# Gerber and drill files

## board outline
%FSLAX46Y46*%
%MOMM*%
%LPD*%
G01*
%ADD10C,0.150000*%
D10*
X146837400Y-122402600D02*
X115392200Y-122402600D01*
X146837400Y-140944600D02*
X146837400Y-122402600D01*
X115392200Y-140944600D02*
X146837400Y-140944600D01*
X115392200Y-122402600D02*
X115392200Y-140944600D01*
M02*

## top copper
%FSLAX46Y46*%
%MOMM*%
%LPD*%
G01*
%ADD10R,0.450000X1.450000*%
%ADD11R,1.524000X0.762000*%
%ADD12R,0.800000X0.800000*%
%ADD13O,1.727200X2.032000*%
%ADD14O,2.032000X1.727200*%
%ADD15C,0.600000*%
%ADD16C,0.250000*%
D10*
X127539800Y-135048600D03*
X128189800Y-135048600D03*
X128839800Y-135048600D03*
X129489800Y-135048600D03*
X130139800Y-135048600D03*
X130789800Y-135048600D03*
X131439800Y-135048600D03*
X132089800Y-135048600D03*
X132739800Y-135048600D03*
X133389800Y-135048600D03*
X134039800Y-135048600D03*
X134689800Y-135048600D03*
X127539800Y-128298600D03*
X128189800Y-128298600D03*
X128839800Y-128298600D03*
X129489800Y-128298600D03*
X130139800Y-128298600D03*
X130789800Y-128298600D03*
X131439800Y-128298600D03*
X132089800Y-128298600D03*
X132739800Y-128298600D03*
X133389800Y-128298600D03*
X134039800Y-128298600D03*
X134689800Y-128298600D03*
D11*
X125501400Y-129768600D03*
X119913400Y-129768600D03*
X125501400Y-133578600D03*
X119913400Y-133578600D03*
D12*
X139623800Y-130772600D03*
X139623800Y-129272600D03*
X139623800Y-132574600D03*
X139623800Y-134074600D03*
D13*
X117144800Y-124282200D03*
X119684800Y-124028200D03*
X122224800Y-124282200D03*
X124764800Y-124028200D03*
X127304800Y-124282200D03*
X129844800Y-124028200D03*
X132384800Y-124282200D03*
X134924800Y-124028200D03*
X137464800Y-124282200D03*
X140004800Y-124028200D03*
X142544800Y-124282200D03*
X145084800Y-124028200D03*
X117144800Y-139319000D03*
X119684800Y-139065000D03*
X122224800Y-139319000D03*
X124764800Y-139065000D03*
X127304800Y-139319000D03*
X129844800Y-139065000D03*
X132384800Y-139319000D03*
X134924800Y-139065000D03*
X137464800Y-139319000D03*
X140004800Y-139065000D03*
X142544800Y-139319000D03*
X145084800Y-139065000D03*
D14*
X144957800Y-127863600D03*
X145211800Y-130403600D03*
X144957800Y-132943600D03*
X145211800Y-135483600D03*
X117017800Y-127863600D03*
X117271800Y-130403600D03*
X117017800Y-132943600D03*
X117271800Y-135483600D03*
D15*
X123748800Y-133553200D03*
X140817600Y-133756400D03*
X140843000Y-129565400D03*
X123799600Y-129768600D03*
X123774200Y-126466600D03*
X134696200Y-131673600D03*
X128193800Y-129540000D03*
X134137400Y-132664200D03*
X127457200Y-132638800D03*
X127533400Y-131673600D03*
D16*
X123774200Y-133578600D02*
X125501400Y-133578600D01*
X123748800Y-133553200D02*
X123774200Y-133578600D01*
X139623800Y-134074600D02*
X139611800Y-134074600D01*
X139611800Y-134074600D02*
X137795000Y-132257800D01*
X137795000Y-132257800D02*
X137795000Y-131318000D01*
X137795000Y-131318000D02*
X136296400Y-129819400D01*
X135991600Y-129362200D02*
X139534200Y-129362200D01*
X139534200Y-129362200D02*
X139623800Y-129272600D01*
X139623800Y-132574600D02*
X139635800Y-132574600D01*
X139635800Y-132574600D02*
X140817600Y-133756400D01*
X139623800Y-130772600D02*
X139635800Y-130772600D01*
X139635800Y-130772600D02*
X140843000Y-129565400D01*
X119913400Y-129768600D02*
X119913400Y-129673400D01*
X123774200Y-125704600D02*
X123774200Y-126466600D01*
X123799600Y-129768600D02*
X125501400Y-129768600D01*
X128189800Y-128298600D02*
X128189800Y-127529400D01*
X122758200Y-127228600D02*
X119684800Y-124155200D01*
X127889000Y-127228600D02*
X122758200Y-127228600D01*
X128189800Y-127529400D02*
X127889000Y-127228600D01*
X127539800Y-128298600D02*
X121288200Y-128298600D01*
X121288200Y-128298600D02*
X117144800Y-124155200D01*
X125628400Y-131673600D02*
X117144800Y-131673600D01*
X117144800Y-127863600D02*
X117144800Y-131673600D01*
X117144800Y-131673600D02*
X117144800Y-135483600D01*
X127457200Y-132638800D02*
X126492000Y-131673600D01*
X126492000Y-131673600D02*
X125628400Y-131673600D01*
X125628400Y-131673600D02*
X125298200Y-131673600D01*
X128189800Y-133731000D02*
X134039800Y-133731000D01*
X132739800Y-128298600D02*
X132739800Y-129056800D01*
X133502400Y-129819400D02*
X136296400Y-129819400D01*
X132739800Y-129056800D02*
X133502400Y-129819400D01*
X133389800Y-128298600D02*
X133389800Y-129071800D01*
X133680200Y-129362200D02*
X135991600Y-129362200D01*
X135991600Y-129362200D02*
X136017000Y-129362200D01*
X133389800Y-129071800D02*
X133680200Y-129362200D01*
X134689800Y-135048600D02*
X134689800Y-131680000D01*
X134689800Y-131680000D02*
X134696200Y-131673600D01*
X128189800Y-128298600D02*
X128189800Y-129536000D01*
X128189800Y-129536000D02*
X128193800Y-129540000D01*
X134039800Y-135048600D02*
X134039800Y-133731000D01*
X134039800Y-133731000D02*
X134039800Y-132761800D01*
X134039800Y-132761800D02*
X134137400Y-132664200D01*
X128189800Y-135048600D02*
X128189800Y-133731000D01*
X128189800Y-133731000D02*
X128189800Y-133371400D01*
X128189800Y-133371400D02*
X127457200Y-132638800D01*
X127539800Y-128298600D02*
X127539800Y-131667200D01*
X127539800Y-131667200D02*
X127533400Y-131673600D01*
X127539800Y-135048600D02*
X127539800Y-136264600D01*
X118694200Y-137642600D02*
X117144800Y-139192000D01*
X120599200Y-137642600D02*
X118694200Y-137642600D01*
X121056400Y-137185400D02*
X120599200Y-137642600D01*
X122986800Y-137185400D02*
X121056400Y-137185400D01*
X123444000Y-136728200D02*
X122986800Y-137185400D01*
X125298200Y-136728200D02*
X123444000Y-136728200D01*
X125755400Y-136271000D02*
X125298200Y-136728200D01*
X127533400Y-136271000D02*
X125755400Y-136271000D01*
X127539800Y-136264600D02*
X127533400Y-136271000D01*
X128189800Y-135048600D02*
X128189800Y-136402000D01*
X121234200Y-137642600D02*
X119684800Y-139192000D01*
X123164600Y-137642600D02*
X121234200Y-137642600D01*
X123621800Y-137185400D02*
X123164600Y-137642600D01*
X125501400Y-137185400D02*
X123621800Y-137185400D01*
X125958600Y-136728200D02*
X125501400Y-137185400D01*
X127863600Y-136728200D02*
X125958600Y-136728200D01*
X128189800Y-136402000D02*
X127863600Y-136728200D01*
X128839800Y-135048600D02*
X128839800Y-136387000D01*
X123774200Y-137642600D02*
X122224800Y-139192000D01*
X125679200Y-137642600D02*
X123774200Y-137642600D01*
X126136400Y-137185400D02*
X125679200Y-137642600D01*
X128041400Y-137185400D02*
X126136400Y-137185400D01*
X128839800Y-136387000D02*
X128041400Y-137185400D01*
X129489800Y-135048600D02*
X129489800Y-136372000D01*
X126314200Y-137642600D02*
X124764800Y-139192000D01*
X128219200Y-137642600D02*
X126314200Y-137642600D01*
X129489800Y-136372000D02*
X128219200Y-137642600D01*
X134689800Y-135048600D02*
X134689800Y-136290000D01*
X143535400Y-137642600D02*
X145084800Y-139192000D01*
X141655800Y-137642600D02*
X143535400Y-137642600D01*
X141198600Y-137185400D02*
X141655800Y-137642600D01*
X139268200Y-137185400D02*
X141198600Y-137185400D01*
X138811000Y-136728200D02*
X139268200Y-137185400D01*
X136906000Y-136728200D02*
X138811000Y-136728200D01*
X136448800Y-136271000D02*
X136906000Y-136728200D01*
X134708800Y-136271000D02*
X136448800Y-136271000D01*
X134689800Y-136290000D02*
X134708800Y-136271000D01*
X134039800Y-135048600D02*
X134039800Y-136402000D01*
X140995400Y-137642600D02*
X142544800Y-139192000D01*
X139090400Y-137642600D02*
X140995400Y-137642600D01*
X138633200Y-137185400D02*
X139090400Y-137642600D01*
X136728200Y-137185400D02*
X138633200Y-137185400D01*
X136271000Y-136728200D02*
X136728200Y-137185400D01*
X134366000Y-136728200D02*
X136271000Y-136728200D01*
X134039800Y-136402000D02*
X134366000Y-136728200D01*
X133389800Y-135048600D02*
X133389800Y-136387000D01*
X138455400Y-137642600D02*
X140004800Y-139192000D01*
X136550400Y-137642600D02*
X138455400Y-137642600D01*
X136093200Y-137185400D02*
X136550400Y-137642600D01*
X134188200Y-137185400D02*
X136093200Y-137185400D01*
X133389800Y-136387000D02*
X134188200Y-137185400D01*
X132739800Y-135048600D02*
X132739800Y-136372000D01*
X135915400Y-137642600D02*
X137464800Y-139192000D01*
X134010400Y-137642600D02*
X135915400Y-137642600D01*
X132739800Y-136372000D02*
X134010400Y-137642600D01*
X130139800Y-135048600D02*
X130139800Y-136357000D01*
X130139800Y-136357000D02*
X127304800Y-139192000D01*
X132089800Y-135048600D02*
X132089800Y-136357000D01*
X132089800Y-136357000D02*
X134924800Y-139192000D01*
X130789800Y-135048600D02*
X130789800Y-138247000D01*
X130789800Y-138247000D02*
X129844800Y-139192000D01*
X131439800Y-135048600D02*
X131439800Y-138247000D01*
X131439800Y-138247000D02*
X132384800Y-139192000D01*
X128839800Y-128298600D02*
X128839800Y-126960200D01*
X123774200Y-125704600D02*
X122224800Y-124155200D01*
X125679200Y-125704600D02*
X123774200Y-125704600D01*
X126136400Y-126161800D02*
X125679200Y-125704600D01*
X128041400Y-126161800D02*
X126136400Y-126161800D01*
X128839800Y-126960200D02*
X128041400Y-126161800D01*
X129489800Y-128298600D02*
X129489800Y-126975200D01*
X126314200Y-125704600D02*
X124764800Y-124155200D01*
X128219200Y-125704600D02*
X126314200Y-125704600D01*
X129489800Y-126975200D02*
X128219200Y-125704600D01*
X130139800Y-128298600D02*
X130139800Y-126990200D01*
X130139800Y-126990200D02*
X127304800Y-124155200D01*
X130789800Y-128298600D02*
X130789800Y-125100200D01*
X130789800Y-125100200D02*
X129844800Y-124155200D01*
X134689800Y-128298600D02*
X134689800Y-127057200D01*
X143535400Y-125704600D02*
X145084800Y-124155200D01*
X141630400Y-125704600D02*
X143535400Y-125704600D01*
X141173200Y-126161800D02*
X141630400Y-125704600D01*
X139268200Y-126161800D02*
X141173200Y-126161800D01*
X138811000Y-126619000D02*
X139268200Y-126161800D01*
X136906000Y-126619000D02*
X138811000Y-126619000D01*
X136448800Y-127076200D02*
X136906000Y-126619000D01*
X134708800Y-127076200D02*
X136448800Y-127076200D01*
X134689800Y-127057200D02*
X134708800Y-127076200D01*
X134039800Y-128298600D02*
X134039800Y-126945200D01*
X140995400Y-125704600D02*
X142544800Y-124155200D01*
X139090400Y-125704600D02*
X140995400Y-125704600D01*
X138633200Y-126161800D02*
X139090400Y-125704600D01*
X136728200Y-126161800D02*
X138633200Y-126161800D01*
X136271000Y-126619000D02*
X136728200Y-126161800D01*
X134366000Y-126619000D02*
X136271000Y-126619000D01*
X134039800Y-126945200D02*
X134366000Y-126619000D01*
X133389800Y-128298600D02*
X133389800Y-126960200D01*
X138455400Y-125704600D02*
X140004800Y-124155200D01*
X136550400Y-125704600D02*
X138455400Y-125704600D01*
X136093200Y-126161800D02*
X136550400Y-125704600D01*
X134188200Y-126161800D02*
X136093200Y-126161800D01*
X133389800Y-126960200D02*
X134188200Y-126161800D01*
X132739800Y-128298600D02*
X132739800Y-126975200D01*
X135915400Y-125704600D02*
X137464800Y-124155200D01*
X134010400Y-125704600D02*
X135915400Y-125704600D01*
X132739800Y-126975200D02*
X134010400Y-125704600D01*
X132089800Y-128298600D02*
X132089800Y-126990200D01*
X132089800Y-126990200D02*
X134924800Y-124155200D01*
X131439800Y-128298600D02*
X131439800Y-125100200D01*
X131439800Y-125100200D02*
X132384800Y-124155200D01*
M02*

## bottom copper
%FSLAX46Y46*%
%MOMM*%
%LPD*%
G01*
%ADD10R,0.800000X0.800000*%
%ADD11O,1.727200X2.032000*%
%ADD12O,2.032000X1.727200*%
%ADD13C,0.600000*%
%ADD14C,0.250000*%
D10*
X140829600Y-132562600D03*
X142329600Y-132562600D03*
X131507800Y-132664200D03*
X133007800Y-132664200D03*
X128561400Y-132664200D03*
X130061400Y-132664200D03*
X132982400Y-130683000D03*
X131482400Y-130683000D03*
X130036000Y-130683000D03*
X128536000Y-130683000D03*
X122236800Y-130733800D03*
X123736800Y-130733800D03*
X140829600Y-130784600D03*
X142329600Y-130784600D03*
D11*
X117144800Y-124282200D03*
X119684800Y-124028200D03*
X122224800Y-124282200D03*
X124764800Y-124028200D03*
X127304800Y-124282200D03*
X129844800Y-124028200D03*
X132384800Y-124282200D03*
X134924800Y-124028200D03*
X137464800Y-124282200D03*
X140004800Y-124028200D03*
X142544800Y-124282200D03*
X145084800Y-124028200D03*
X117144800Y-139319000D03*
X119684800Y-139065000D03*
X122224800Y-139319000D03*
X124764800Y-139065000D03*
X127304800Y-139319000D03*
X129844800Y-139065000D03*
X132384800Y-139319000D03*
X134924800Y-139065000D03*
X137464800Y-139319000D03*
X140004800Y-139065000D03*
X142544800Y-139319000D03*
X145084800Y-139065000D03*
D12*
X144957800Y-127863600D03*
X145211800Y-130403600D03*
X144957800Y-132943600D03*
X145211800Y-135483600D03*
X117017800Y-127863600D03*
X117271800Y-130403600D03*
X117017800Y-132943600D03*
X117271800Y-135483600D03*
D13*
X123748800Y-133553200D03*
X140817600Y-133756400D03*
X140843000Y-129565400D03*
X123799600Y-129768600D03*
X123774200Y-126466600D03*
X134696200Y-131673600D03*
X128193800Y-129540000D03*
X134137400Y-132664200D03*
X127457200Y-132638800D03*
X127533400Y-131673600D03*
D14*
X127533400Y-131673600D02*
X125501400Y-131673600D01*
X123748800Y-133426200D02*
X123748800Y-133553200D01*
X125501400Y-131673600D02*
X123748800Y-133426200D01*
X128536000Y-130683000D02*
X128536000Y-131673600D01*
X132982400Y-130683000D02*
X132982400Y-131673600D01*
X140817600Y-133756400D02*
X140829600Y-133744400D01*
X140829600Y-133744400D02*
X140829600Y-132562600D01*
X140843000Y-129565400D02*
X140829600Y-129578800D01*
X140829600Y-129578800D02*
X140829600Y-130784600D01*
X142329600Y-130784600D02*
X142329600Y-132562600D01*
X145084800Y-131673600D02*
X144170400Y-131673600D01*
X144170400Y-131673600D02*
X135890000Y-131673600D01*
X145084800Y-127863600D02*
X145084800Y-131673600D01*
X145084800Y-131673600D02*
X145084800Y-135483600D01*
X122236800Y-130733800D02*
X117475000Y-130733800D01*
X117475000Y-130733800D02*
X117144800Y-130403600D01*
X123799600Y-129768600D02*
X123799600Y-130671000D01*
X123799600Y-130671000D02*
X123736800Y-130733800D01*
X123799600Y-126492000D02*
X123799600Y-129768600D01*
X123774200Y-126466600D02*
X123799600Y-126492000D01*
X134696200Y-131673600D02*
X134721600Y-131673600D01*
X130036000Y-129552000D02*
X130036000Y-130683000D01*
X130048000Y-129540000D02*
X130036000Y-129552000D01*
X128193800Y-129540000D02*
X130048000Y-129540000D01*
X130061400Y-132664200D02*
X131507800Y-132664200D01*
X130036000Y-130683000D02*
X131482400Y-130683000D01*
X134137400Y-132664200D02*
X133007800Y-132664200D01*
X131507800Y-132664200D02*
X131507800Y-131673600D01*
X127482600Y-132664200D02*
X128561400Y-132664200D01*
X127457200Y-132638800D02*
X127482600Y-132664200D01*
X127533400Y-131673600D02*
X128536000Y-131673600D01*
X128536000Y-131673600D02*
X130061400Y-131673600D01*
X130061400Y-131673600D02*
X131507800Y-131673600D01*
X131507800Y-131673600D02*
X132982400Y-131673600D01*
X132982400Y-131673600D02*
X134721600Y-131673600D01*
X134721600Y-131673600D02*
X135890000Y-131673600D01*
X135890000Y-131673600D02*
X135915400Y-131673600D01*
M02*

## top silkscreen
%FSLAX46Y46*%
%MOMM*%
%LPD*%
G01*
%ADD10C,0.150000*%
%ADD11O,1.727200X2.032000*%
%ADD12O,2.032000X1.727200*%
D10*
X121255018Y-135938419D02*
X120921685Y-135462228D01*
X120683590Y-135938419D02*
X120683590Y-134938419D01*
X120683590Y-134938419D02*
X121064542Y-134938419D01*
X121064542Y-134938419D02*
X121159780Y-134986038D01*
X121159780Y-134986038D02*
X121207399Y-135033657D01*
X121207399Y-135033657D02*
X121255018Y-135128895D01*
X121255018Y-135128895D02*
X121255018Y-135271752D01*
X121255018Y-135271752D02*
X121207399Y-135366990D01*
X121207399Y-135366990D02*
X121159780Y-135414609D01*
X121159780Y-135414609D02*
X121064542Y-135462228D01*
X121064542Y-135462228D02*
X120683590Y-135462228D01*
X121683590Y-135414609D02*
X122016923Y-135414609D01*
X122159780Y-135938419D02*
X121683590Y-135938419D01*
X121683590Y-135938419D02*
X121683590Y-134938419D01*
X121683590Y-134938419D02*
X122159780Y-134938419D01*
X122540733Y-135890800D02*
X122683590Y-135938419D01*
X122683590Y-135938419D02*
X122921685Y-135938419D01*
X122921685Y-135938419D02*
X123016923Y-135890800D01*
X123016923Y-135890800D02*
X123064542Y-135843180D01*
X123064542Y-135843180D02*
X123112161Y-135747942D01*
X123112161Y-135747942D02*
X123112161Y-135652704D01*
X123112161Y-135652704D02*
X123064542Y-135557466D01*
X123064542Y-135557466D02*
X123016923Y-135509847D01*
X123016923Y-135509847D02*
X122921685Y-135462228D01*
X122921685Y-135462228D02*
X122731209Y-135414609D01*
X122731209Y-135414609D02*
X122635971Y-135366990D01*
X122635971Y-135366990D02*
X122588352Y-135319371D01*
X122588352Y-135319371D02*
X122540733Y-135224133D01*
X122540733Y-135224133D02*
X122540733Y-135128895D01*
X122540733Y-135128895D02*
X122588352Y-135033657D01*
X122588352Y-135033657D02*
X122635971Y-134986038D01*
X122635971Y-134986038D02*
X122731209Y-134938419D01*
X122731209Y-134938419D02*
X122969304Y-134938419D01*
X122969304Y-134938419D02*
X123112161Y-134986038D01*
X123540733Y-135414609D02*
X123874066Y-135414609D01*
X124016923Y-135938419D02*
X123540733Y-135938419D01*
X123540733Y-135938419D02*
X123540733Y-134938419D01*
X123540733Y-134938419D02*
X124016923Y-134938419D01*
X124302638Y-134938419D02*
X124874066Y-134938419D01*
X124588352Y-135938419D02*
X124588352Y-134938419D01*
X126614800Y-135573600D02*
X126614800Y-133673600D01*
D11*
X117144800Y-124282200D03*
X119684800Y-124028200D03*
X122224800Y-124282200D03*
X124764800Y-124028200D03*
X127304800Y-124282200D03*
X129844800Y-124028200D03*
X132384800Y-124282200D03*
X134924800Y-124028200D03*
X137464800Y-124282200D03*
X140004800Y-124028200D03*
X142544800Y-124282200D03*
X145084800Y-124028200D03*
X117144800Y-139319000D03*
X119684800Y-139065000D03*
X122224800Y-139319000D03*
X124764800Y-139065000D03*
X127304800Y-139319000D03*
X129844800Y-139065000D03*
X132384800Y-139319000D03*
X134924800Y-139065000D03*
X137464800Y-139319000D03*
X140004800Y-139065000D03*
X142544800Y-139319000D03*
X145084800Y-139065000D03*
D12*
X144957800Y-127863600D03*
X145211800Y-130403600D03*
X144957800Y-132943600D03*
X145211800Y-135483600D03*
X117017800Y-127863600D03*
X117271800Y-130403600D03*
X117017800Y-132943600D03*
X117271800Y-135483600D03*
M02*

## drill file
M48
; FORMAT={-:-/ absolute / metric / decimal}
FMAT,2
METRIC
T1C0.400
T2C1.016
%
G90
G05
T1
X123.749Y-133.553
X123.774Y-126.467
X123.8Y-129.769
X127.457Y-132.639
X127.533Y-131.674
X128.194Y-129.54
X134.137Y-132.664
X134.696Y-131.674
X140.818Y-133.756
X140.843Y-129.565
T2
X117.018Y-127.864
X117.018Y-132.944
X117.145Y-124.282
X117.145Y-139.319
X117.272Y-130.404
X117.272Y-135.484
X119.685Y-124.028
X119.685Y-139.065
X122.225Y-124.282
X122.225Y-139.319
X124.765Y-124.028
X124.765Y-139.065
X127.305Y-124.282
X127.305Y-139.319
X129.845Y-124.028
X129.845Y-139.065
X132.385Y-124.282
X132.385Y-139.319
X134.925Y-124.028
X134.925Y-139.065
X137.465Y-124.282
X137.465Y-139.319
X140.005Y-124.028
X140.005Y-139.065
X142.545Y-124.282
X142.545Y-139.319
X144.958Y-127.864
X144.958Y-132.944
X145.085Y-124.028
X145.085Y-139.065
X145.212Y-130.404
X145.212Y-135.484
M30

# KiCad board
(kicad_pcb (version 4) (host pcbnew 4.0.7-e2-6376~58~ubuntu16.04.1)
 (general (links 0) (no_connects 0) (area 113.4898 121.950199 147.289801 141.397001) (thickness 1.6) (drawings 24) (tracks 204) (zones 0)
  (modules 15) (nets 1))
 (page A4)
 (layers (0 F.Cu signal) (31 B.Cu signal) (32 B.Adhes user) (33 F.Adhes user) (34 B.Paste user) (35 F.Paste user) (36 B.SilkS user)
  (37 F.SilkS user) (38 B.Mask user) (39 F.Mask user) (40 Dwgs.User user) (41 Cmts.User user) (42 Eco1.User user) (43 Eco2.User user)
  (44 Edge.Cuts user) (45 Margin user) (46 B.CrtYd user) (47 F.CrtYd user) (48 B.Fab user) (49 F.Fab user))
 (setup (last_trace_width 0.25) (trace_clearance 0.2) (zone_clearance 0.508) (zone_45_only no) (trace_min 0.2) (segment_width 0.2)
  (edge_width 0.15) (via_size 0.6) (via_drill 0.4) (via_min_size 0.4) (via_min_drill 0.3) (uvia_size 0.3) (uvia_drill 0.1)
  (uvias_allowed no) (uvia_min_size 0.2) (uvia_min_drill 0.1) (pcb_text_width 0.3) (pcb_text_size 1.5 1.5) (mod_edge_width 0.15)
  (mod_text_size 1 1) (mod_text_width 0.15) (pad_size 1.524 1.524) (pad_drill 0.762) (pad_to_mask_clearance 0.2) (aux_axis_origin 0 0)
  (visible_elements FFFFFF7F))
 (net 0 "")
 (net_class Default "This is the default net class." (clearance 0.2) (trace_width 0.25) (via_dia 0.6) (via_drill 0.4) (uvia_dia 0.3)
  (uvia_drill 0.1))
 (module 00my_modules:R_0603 (layer B.Cu) (at 141.5796 132.5626)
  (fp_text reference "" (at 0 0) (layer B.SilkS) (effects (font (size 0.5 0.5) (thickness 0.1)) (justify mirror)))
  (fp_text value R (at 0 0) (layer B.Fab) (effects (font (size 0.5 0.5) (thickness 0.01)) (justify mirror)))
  (pad 1 smd rect (at -0.75 0) (size 0.8 0.8) (layers B.Cu B.Paste B.Mask))
  (pad 2 smd rect (at 0.75 0) (size 0.8 0.8) (layers B.Cu B.Paste B.Mask)))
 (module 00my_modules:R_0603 (layer B.Cu) (at 132.2578 132.6642)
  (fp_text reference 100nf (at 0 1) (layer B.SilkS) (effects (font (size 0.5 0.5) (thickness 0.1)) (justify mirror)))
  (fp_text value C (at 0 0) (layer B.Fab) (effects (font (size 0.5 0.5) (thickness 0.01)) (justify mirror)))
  (pad 1 smd rect (at -0.75 0) (size 0.8 0.8) (layers B.Cu B.Paste B.Mask))
  (pad 2 smd rect (at 0.75 0) (size 0.8 0.8) (layers B.Cu B.Paste B.Mask)))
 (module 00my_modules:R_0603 (layer B.Cu) (at 129.3114 132.6642)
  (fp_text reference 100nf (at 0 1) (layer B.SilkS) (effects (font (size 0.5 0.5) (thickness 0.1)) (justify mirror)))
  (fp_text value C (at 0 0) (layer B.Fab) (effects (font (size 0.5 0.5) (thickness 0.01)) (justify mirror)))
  (pad 1 smd rect (at -0.75 0) (size 0.8 0.8) (layers B.Cu B.Paste B.Mask))
  (pad 2 smd rect (at 0.75 0) (size 0.8 0.8) (layers B.Cu B.Paste B.Mask)))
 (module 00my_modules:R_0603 (layer B.Cu) (at 132.2324 130.683 180)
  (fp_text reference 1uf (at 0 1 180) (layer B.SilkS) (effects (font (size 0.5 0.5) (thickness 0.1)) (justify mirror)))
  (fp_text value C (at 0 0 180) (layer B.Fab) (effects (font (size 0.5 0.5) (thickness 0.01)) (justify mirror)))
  (pad 1 smd rect (at -0.75 0 180) (size 0.8 0.8) (layers B.Cu B.Paste B.Mask))
  (pad 2 smd rect (at 0.75 0 180) (size 0.8 0.8) (layers B.Cu B.Paste B.Mask)))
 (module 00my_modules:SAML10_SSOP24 (layer F.Cu) (at 131.1148 131.6736 90)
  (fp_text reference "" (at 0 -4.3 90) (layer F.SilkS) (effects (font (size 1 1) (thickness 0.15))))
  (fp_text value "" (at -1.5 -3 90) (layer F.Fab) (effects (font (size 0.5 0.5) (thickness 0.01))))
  (fp_line (start -3.9 -4.5) (end -2 -4.5) (layer F.SilkS) (width 0.15))
  (pad VOUT smd rect (at -3.375 -3.575 90) (size 1.45 0.45) (layers F.Cu F.Paste F.Mask))
  (pad VIO smd rect (at -3.375 -2.925 90) (size 1.45 0.45) (layers F.Cu F.Paste F.Mask))
  (pad SWCL smd rect (at -3.375 -2.275 90) (size 1.45 0.45) (layers F.Cu F.Paste F.Mask))
  (pad SWDI smd rect (at -3.375 -1.625 90) (size 1.45 0.45) (layers F.Cu F.Paste F.Mask))
  (pad PA00 smd rect (at -3.375 -0.975 90) (size 1.45 0.45) (layers F.Cu F.Paste F.Mask))
  (pad PA01 smd rect (at -3.375 -0.325 90) (size 1.45 0.45) (layers F.Cu F.Paste F.Mask))
  (pad PA02 smd rect (at -3.375 0.325 90) (size 1.45 0.45) (layers F.Cu F.Paste F.Mask))
  (pad PA03 smd rect (at -3.375 0.975 90) (size 1.45 0.45) (layers F.Cu F.Paste F.Mask))
  (pad PA04 smd rect (at -3.375 1.625 90) (size 1.45 0.45) (layers F.Cu F.Paste F.Mask))
  (pad PA05 smd rect (at -3.375 2.275 90) (size 1.45 0.45) (layers F.Cu F.Paste F.Mask))
  (pad VANA smd rect (at -3.375 2.925 90) (size 1.45 0.45) (layers F.Cu F.Paste F.Mask))
  (pad GANA smd rect (at -3.375 3.575 90) (size 1.45 0.45) (layers F.Cu F.Paste F.Mask))
  (pad GND smd rect (at 3.375 -3.575 90) (size 1.45 0.45) (layers F.Cu F.Paste F.Mask))
  (pad VCOR smd rect (at 3.375 -2.925 90) (size 1.45 0.45) (layers F.Cu F.Paste F.Mask))
  (pad RSTN smd rect (at 3.375 -2.275 90) (size 1.45 0.45) (layers F.Cu F.Paste F.Mask))
  (pad PA23 smd rect (at 3.375 -1.625 90) (size 1.45 0.45) (layers F.Cu F.Paste F.Mask))
  (pad PA22 smd rect (at 3.375 -0.975 90) (size 1.45 0.45) (layers F.Cu F.Paste F.Mask))
  (pad PA19 smd rect (at 3.375 -0.325 90) (size 1.45 0.45) (layers F.Cu F.Paste F.Mask))
  (pad PA18 smd rect (at 3.375 0.325 90) (size 1.45 0.45) (layers F.Cu F.Paste F.Mask))
  (pad PA17 smd rect (at 3.375 0.975 90) (size 1.45 0.45) (layers F.Cu F.Paste F.Mask))
  (pad PA16 smd rect (at 3.375 1.625 90) (size 1.45 0.45) (layers F.Cu F.Paste F.Mask))
  (pad PA15 smd rect (at 3.375 2.275 90) (size 1.45 0.45) (layers F.Cu F.Paste F.Mask))
  (pad PA14 smd rect (at 3.375 2.925 90) (size 1.45 0.45) (layers F.Cu F.Paste F.Mask))
  (pad PA08 smd rect (at 3.375 3.575 90) (size 1.45 0.45) (layers F.Cu F.Paste F.Mask)))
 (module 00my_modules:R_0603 (layer B.Cu) (at 129.286 130.683 180)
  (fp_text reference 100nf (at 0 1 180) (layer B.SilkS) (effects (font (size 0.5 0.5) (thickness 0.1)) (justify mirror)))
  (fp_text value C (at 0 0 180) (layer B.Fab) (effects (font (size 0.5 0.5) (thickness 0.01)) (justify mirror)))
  (pad 1 smd rect (at -0.75 0 180) (size 0.8 0.8) (layers B.Cu B.Paste B.Mask))
  (pad 2 smd rect (at 0.75 0 180) (size 0.8 0.8) (layers B.Cu B.Paste B.Mask)))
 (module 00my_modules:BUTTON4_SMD (layer F.Cu) (at 122.7074 131.6736 180)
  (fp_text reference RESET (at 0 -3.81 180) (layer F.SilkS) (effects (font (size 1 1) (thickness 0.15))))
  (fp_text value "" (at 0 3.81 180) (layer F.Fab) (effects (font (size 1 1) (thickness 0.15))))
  (pad 1 smd rect (at -2.794 1.905 180) (size 1.524 0.762) (layers F.Cu F.Paste F.Mask))
  (pad 2 smd rect (at 2.794 1.905 180) (size 1.524 0.762) (layers F.Cu F.Paste F.Mask))
  (pad 3 smd rect (at -2.794 -1.905 180) (size 1.524 0.762) (layers F.Cu F.Paste F.Mask))
  (pad 4 smd rect (at 2.794 -1.905 180) (size 1.524 0.762) (layers F.Cu F.Paste F.Mask)))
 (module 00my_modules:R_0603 (layer B.Cu) (at 122.9868 130.7338)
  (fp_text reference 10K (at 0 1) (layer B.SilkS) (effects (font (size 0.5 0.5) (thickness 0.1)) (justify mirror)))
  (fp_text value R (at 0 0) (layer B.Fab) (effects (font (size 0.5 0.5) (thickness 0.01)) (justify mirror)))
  (pad 1 smd rect (at -0.75 0) (size 0.8 0.8) (layers B.Cu B.Paste B.Mask))
  (pad 2 smd rect (at 0.75 0) (size 0.8 0.8) (layers B.Cu B.Paste B.Mask)))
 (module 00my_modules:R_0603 (layer B.Cu) (at 141.5796 130.7846)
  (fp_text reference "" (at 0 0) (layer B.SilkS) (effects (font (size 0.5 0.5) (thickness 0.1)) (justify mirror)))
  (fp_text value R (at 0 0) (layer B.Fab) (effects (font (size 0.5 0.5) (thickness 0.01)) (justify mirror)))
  (pad 1 smd rect (at -0.75 0) (size 0.8 0.8) (layers B.Cu B.Paste B.Mask))
  (pad 2 smd rect (at 0.75 0) (size 0.8 0.8) (layers B.Cu B.Paste B.Mask)))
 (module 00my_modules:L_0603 (layer F.Cu) (at 139.6238 130.0226 90)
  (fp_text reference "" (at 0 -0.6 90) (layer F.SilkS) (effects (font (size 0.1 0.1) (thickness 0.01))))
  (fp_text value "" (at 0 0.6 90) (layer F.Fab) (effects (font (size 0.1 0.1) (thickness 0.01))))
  (pad 1 smd rect (at -0.75 0 90) (size 0.8 0.8) (layers F.Cu F.Paste F.Mask))
  (pad 2 smd rect (at 0.75 0 90) (size 0.8 0.8) (layers F.Cu F.Paste F.Mask)))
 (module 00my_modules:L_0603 (layer F.Cu) (at 139.6238 133.3246 270)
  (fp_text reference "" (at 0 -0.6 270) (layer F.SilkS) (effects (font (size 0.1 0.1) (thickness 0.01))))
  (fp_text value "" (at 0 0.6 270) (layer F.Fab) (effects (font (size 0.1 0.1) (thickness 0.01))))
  (pad 1 smd rect (at -0.75 0 270) (size 0.8 0.8) (layers F.Cu F.Paste F.Mask))
  (pad 2 smd rect (at 0.75 0 270) (size 0.8 0.8) (layers F.Cu F.Paste F.Mask)))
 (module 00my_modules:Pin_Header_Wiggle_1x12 (layer F.Cu) (at 117.1448 124.1552 90)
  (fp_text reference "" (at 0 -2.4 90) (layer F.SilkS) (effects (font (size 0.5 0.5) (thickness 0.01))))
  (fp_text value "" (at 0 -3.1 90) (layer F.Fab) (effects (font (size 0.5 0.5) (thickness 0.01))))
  (pad 1 thru_hole oval (at -0.127 0 90) (size 2.032 1.7272) (drill 1.016) (layers *.Cu *.Mask F.SilkS))
  (pad 2 thru_hole oval (at 0.127 2.54 90) (size 2.032 1.7272) (drill 1.016) (layers *.Cu *.Mask F.SilkS))
  (pad 3 thru_hole oval (at -0.127 5.08 90) (size 2.032 1.7272) (drill 1.016) (layers *.Cu *.Mask F.SilkS))
  (pad 4 thru_hole oval (at 0.127 7.62 90) (size 2.032 1.7272) (drill 1.016) (layers *.Cu *.Mask F.SilkS))
  (pad 5 thru_hole oval (at -0.127 10.16 90) (size 2.032 1.7272) (drill 1.016) (layers *.Cu *.Mask F.SilkS))
  (pad 6 thru_hole oval (at 0.127 12.7 90) (size 2.032 1.7272) (drill 1.016) (layers *.Cu *.Mask F.SilkS))
  (pad 7 thru_hole oval (at -0.127 15.24 90) (size 2.032 1.7272) (drill 1.016) (layers *.Cu *.Mask F.SilkS))
  (pad 8 thru_hole oval (at 0.127 17.78 90) (size 2.032 1.7272) (drill 1.016) (layers *.Cu *.Mask F.SilkS))
  (pad 9 thru_hole oval (at -0.127 20.32 90) (size 2.032 1.7272) (drill 1.016) (layers *.Cu *.Mask F.SilkS))
  (pad 10 thru_hole oval (at 0.127 22.86 90) (size 2.032 1.7272) (drill 1.016) (layers *.Cu *.Mask F.SilkS))
  (pad 11 thru_hole oval (at -0.127 25.4 90) (size 2.032 1.7272) (drill 1.016) (layers *.Cu *.Mask F.SilkS))
  (pad 12 thru_hole oval (at 0.127 27.94 90) (size 2.032 1.7272) (drill 1.016) (layers *.Cu *.Mask F.SilkS)))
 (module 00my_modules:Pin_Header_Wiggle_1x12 (layer F.Cu) (at 117.1448 139.192 90)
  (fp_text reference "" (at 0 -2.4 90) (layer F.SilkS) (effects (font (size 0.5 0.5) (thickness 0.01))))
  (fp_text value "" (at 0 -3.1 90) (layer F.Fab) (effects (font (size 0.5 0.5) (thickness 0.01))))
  (pad 1 thru_hole oval (at -0.127 0 90) (size 2.032 1.7272) (drill 1.016) (layers *.Cu *.Mask F.SilkS))
  (pad 2 thru_hole oval (at 0.127 2.54 90) (size 2.032 1.7272) (drill 1.016) (layers *.Cu *.Mask F.SilkS))
  (pad 3 thru_hole oval (at -0.127 5.08 90) (size 2.032 1.7272) (drill 1.016) (layers *.Cu *.Mask F.SilkS))
  (pad 4 thru_hole oval (at 0.127 7.62 90) (size 2.032 1.7272) (drill 1.016) (layers *.Cu *.Mask F.SilkS))
  (pad 5 thru_hole oval (at -0.127 10.16 90) (size 2.032 1.7272) (drill 1.016) (layers *.Cu *.Mask F.SilkS))
  (pad 6 thru_hole oval (at 0.127 12.7 90) (size 2.032 1.7272) (drill 1.016) (layers *.Cu *.Mask F.SilkS))
  (pad 7 thru_hole oval (at -0.127 15.24 90) (size 2.032 1.7272) (drill 1.016) (layers *.Cu *.Mask F.SilkS))
  (pad 8 thru_hole oval (at 0.127 17.78 90) (size 2.032 1.7272) (drill 1.016) (layers *.Cu *.Mask F.SilkS))
  (pad 9 thru_hole oval (at -0.127 20.32 90) (size 2.032 1.7272) (drill 1.016) (layers *.Cu *.Mask F.SilkS))
  (pad 10 thru_hole oval (at 0.127 22.86 90) (size 2.032 1.7272) (drill 1.016) (layers *.Cu *.Mask F.SilkS))
  (pad 11 thru_hole oval (at -0.127 25.4 90) (size 2.032 1.7272) (drill 1.016) (layers *.Cu *.Mask F.SilkS))
  (pad 12 thru_hole oval (at 0.127 27.94 90) (size 2.032 1.7272) (drill 1.016) (layers *.Cu *.Mask F.SilkS)))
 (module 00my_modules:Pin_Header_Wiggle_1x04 (layer F.Cu) (at 145.0848 127.8636)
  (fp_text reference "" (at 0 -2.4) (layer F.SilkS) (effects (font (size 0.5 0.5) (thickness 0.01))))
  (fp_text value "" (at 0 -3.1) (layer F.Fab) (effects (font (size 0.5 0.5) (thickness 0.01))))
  (pad 1 thru_hole oval (at -0.127 0) (size 2.032 1.7272) (drill 1.016) (layers *.Cu *.Mask F.SilkS))
  (pad 2 thru_hole oval (at 0.127 2.54) (size 2.032 1.7272) (drill 1.016) (layers *.Cu *.Mask F.SilkS))
  (pad 3 thru_hole oval (at -0.127 5.08) (size 2.032 1.7272) (drill 1.016) (layers *.Cu *.Mask F.SilkS))
  (pad 4 thru_hole oval (at 0.127 7.62) (size 2.032 1.7272) (drill 1.016) (layers *.Cu *.Mask F.SilkS)))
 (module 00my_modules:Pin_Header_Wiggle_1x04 (layer F.Cu) (at 117.1448 127.8636)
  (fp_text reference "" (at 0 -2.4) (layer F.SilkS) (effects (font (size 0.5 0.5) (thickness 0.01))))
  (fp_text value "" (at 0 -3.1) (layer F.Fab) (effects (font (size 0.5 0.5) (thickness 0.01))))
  (pad 1 thru_hole oval (at -0.127 0) (size 2.032 1.7272) (drill 1.016) (layers *.Cu *.Mask F.SilkS))
  (pad 2 thru_hole oval (at 0.127 2.54) (size 2.032 1.7272) (drill 1.016) (layers *.Cu *.Mask F.SilkS))
  (pad 3 thru_hole oval (at -0.127 5.08) (size 2.032 1.7272) (drill 1.016) (layers *.Cu *.Mask F.SilkS))
  (pad 4 thru_hole oval (at 0.127 7.62) (size 2.032 1.7272) (drill 1.016) (layers *.Cu *.Mask F.SilkS)))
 (gr_line (start 146.8374 122.4026) (end 115.3922 122.4026) (angle 90) (layer Edge.Cuts) (width 0.15))
 (gr_line (start 146.8374 140.9446) (end 146.8374 122.4026) (angle 90) (layer Edge.Cuts) (width 0.15))
 (gr_line (start 115.3922 140.9446) (end 146.8374 140.9446) (angle 90) (layer Edge.Cuts) (width 0.15))
 (gr_line (start 115.3922 122.4026) (end 115.3922 140.9446) (angle 90) (layer Edge.Cuts) (width 0.15))
 (segment (start 127.5334 131.6736) (end 125.5014 131.6736) (width 0.25) (layer B.Cu) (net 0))
 (segment (start 123.7742 133.5786) (end 125.5014 133.5786) (width 0.25) (layer F.Cu) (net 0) (status 800000))
 (segment (start 123.7488 133.5532) (end 123.7742 133.5786) (width 0.25) (layer F.Cu) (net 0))
 (via (at 123.7488 133.5532) (size 0.6) (drill 0.4) (layers F.Cu B.Cu) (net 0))
 (segment (start 123.7488 133.4262) (end 123.7488 133.5532) (width 0.25) (layer B.Cu) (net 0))
 (segment (start 125.5014 131.6736) (end 123.7488 133.4262) (width 0.25) (layer B.Cu) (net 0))
 (segment (start 128.536 130.683) (end 128.536 131.6736) (width 0.25) (layer B.Cu) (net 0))
 (segment (start 132.9824 130.683) (end 132.9824 131.6736) (width 0.25) (layer B.Cu) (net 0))
 (segment (start 139.6238 134.0746) (end 139.6118 134.0746) (width 0.25) (layer F.Cu) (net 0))
 (segment (start 139.6118 134.0746) (end 137.795 132.2578) (width 0.25) (layer F.Cu) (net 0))
 (segment (start 137.795 132.2578) (end 137.795 131.318) (width 0.25) (layer F.Cu) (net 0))
 (segment (start 137.795 131.318) (end 136.2964 129.8194) (width 0.25) (layer F.Cu) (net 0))
 (segment (start 135.9916 129.3622) (end 139.5342 129.3622) (width 0.25) (layer F.Cu) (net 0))
 (segment (start 139.5342 129.3622) (end 139.6238 129.2726) (width 0.25) (layer F.Cu) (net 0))
 (segment (start 139.6238 132.5746) (end 139.6358 132.5746) (width 0.25) (layer F.Cu) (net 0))
 (segment (start 139.6358 132.5746) (end 140.8176 133.7564) (width 0.25) (layer F.Cu) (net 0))
 (via (at 140.8176 133.7564) (size 0.6) (drill 0.4) (layers F.Cu B.Cu) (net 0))
 (segment (start 140.8176 133.7564) (end 140.8296 133.7444) (width 0.25) (layer B.Cu) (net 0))
 (segment (start 140.8296 133.7444) (end 140.8296 132.5626) (width 0.25) (layer B.Cu) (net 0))
 (segment (start 139.6238 130.7726) (end 139.6358 130.7726) (width 0.25) (layer F.Cu) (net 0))
 (segment (start 139.6358 130.7726) (end 140.843 129.5654) (width 0.25) (layer F.Cu) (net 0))
 (via (at 140.843 129.5654) (size 0.6) (drill 0.4) (layers F.Cu B.Cu) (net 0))
 (segment (start 140.843 129.5654) (end 140.8296 129.5788) (width 0.25) (layer B.Cu) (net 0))
 (segment (start 140.8296 129.5788) (end 140.8296 130.7846) (width 0.25) (layer B.Cu) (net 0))
 (segment (start 142.3296 130.7846) (end 142.3296 132.5626) (width 0.25) (layer B.Cu) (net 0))
 (segment (start 145.0848 131.6736) (end 144.1704 131.6736) (width 0.25) (layer B.Cu) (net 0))
 (segment (start 144.1704 131.6736) (end 135.89 131.6736) (width 0.25) (layer B.Cu) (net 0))
 (segment (start 145.0848 127.8636) (end 145.0848 131.6736) (width 0.25) (layer B.Cu) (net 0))
 (segment (start 145.0848 131.6736) (end 145.0848 135.4836) (width 0.25) (layer B.Cu) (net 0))
 (segment (start 122.2368 130.7338) (end 117.475 130.7338) (width 0.25) (layer B.Cu) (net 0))
 (segment (start 117.475 130.7338) (end 117.1448 130.4036) (width 0.25) (layer B.Cu) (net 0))
 (segment (start 123.7996 129.7686) (end 123.7996 130.671) (width 0.25) (layer B.Cu) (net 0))
 (segment (start 123.7996 130.671) (end 123.7368 130.7338) (width 0.25) (layer B.Cu) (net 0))
 (segment (start 119.9134 129.7686) (end 119.9134 129.6734) (width 0.25) (layer F.Cu) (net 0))
 (segment (start 123.7742 125.7046) (end 123.7742 126.4666) (width 0.25) (layer F.Cu) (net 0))
 (segment (start 123.7996 129.7686) (end 125.5014 129.7686) (width 0.25) (layer F.Cu) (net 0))
 (via (at 123.7996 129.7686) (size 0.6) (drill 0.4) (layers F.Cu B.Cu) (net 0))
 (segment (start 123.7996 126.492) (end 123.7996 129.7686) (width 0.25) (layer B.Cu) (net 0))
 (segment (start 123.7742 126.4666) (end 123.7996 126.492) (width 0.25) (layer B.Cu) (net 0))
 (via (at 123.7742 126.4666) (size 0.6) (drill 0.4) (layers F.Cu B.Cu) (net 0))
 (segment (start 128.1898 128.2986) (end 128.1898 127.5294) (width 0.25) (layer F.Cu) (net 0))
 (segment (start 122.7582 127.2286) (end 119.6848 124.1552) (width 0.25) (layer F.Cu) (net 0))
 (segment (start 127.889 127.2286) (end 122.7582 127.2286) (width 0.25) (layer F.Cu) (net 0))
 (segment (start 128.1898 127.5294) (end 127.889 127.2286) (width 0.25) (layer F.Cu) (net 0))
 (segment (start 127.5398 128.2986) (end 121.2882 128.2986) (width 0.25) (layer F.Cu) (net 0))
 (segment (start 121.2882 128.2986) (end 117.1448 124.1552) (width 0.25) (layer F.Cu) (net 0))
 (segment (start 125.6284 131.6736) (end 117.1448 131.6736) (width 0.25) (layer F.Cu) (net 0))
 (segment (start 117.1448 127.8636) (end 117.1448 131.6736) (width 0.25) (layer F.Cu) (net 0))
 (segment (start 117.1448 131.6736) (end 117.1448 135.4836) (width 0.25) (layer F.Cu) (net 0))
 (segment (start 127.4572 132.6388) (end 126.492 131.6736) (width 0.25) (layer F.Cu) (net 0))
 (segment (start 126.492 131.6736) (end 125.6284 131.6736) (width 0.25) (layer F.Cu) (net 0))
 (segment (start 125.6284 131.6736) (end 125.2982 131.6736) (width 0.25) (layer F.Cu) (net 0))
 (segment (start 128.1898 133.731) (end 134.0398 133.731) (width 0.25) (layer F.Cu) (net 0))
 (segment (start 132.7398 128.2986) (end 132.7398 129.0568) (width 0.25) (layer F.Cu) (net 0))
 (segment (start 133.5024 129.8194) (end 136.2964 129.8194) (width 0.25) (layer F.Cu) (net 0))
 (segment (start 132.7398 129.0568) (end 133.5024 129.8194) (width 0.25) (layer F.Cu) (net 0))
 (segment (start 133.3898 128.2986) (end 133.3898 129.0718) (width 0.25) (layer F.Cu) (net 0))
 (segment (start 133.6802 129.3622) (end 135.9916 129.3622) (width 0.25) (layer F.Cu) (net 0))
 (segment (start 135.9916 129.3622) (end 136.017 129.3622) (width 0.25) (layer F.Cu) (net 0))
 (segment (start 133.3898 129.0718) (end 133.6802 129.3622) (width 0.25) (layer F.Cu) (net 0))
 (segment (start 134.6898 135.0486) (end 134.6898 131.68) (width 0.25) (layer F.Cu) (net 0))
 (segment (start 134.6962 131.6736) (end 134.7216 131.6736) (width 0.25) (layer B.Cu) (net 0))
 (via (at 134.6962 131.6736) (size 0.6) (drill 0.4) (layers F.Cu B.Cu) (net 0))
 (segment (start 134.6898 131.68) (end 134.6962 131.6736) (width 0.25) (layer F.Cu) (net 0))
 (segment (start 128.1898 128.2986) (end 128.1898 129.536) (width 0.25) (layer F.Cu) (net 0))
 (segment (start 130.036 129.552) (end 130.036 130.683) (width 0.25) (layer B.Cu) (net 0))
 (segment (start 130.048 129.54) (end 130.036 129.552) (width 0.25) (layer B.Cu) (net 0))
 (segment (start 128.1938 129.54) (end 130.048 129.54) (width 0.25) (layer B.Cu) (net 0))
 (via (at 128.1938 129.54) (size 0.6) (drill 0.4) (layers F.Cu B.Cu) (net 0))
 (segment (start 128.1898 129.536) (end 128.1938 129.54) (width 0.25) (layer F.Cu) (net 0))
 (segment (start 130.0614 132.6642) (end 131.5078 132.6642) (width 0.25) (layer B.Cu) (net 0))
 (segment (start 130.036 130.683) (end 131.4824 130.683) (width 0.25) (layer B.Cu) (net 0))
 (segment (start 134.0398 135.0486) (end 134.0398 133.731) (width 0.25) (layer F.Cu) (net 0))
 (segment (start 134.0398 133.731) (end 134.0398 132.7618) (width 0.25) (layer F.Cu) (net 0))
 (segment (start 134.0398 132.7618) (end 134.1374 132.6642) (width 0.25) (layer F.Cu) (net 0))
 (via (at 134.1374 132.6642) (size 0.6) (drill 0.4) (layers F.Cu B.Cu) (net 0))
 (segment (start 134.1374 132.6642) (end 133.0078 132.6642) (width 0.25) (layer B.Cu) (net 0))
 (segment (start 131.5078 132.6642) (end 131.5078 131.6736) (width 0.25) (layer B.Cu) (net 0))
 (segment (start 128.1898 135.0486) (end 128.1898 133.731) (width 0.25) (layer F.Cu) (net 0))
 (segment (start 128.1898 133.731) (end 128.1898 133.3714) (width 0.25) (layer F.Cu) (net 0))
 (segment (start 127.4826 132.6642) (end 128.5614 132.6642) (width 0.25) (layer B.Cu) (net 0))
 (segment (start 127.4572 132.6388) (end 127.4826 132.6642) (width 0.25) (layer B.Cu) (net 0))
 (via (at 127.4572 132.6388) (size 0.6) (drill 0.4) (layers F.Cu B.Cu) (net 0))
 (segment (start 128.1898 133.3714) (end 127.4572 132.6388) (width 0.25) (layer F.Cu) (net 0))
 (segment (start 127.5398 128.2986) (end 127.5398 131.6672) (width 0.25) (layer F.Cu) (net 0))
 (segment (start 127.5334 131.6736) (end 128.536 131.6736) (width 0.25) (layer B.Cu) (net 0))
 (segment (start 128.536 131.6736) (end 130.0614 131.6736) (width 0.25) (layer B.Cu) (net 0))
 (segment (start 130.0614 131.6736) (end 131.5078 131.6736) (width 0.25) (layer B.Cu) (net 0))
 (segment (start 131.5078 131.6736) (end 132.9824 131.6736) (width 0.25) (layer B.Cu) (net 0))
 (segment (start 132.9824 131.6736) (end 134.7216 131.6736) (width 0.25) (layer B.Cu) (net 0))
 (segment (start 134.7216 131.6736) (end 135.89 131.6736) (width 0.25) (layer B.Cu) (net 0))
 (segment (start 135.89 131.6736) (end 135.9154 131.6736) (width 0.25) (layer B.Cu) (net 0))
 (via (at 127.5334 131.6736) (size 0.6) (drill 0.4) (layers F.Cu B.Cu) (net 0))
 (segment (start 127.5398 131.6672) (end 127.5334 131.6736) (width 0.25) (layer F.Cu) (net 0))
 (segment (start 127.5398 135.0486) (end 127.5398 136.2646) (width 0.25) (layer F.Cu) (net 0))
 (segment (start 118.6942 137.6426) (end 117.1448 139.192) (width 0.25) (layer F.Cu) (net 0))
 (segment (start 120.5992 137.6426) (end 118.6942 137.6426) (width 0.25) (layer F.Cu) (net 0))
 (segment (start 121.0564 137.1854) (end 120.5992 137.6426) (width 0.25) (layer F.Cu) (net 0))
 (segment (start 122.9868 137.1854) (end 121.0564 137.1854) (width 0.25) (layer F.Cu) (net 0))
 (segment (start 123.444 136.7282) (end 122.9868 137.1854) (width 0.25) (layer F.Cu) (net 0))
 (segment (start 125.2982 136.7282) (end 123.444 136.7282) (width 0.25) (layer F.Cu) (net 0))
 (segment (start 125.7554 136.271) (end 125.2982 136.7282) (width 0.25) (layer F.Cu) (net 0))
 (segment (start 127.5334 136.271) (end 125.7554 136.271) (width 0.25) (layer F.Cu) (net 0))
 (segment (start 127.5398 136.2646) (end 127.5334 136.271) (width 0.25) (layer F.Cu) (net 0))
 (segment (start 128.1898 135.0486) (end 128.1898 136.402) (width 0.25) (layer F.Cu) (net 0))
 (segment (start 121.2342 137.6426) (end 119.6848 139.192) (width 0.25) (layer F.Cu) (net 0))
 (segment (start 123.1646 137.6426) (end 121.2342 137.6426) (width 0.25) (layer F.Cu) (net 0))
 (segment (start 123.6218 137.1854) (end 123.1646 137.6426) (width 0.25) (layer F.Cu) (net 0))
 (segment (start 125.5014 137.1854) (end 123.6218 137.1854) (width 0.25) (layer F.Cu) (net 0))
 (segment (start 125.9586 136.7282) (end 125.5014 137.1854) (width 0.25) (layer F.Cu) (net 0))
 (segment (start 127.8636 136.7282) (end 125.9586 136.7282) (width 0.25) (layer F.Cu) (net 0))
 (segment (start 128.1898 136.402) (end 127.8636 136.7282) (width 0.25) (layer F.Cu) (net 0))
 (segment (start 128.8398 135.0486) (end 128.8398 136.387) (width 0.25) (layer F.Cu) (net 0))
 (segment (start 123.7742 137.6426) (end 122.2248 139.192) (width 0.25) (layer F.Cu) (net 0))
 (segment (start 125.6792 137.6426) (end 123.7742 137.6426) (width 0.25) (layer F.Cu) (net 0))
 (segment (start 126.1364 137.1854) (end 125.6792 137.6426) (width 0.25) (layer F.Cu) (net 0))
 (segment (start 128.0414 137.1854) (end 126.1364 137.1854) (width 0.25) (layer F.Cu) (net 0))
 (segment (start 128.8398 136.387) (end 128.0414 137.1854) (width 0.25) (layer F.Cu) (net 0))
 (segment (start 129.4898 135.0486) (end 129.4898 136.372) (width 0.25) (layer F.Cu) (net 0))
 (segment (start 126.3142 137.6426) (end 124.7648 139.192) (width 0.25) (layer F.Cu) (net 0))
 (segment (start 128.2192 137.6426) (end 126.3142 137.6426) (width 0.25) (layer F.Cu) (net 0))
 (segment (start 129.4898 136.372) (end 128.2192 137.6426) (width 0.25) (layer F.Cu) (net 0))
 (segment (start 134.6898 135.0486) (end 134.6898 136.29) (width 0.25) (layer F.Cu) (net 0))
 (segment (start 143.5354 137.6426) (end 145.0848 139.192) (width 0.25) (layer F.Cu) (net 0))
 (segment (start 141.6558 137.6426) (end 143.5354 137.6426) (width 0.25) (layer F.Cu) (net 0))
 (segment (start 141.1986 137.1854) (end 141.6558 137.6426) (width 0.25) (layer F.Cu) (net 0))
 (segment (start 139.2682 137.1854) (end 141.1986 137.1854) (width 0.25) (layer F.Cu) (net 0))
 (segment (start 138.811 136.7282) (end 139.2682 137.1854) (width 0.25) (layer F.Cu) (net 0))
 (segment (start 136.906 136.7282) (end 138.811 136.7282) (width 0.25) (layer F.Cu) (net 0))
 (segment (start 136.4488 136.271) (end 136.906 136.7282) (width 0.25) (layer F.Cu) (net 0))
 (segment (start 134.7088 136.271) (end 136.4488 136.271) (width 0.25) (layer F.Cu) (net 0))
 (segment (start 134.6898 136.29) (end 134.7088 136.271) (width 0.25) (layer F.Cu) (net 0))
 (segment (start 134.0398 135.0486) (end 134.0398 136.402) (width 0.25) (layer F.Cu) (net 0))
 (segment (start 140.9954 137.6426) (end 142.5448 139.192) (width 0.25) (layer F.Cu) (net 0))
 (segment (start 139.0904 137.6426) (end 140.9954 137.6426) (width 0.25) (layer F.Cu) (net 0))
 (segment (start 138.6332 137.1854) (end 139.0904 137.6426) (width 0.25) (layer F.Cu) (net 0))
 (segment (start 136.7282 137.1854) (end 138.6332 137.1854) (width 0.25) (layer F.Cu) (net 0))
 (segment (start 136.271 136.7282) (end 136.7282 137.1854) (width 0.25) (layer F.Cu) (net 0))
 (segment (start 134.366 136.7282) (end 136.271 136.7282) (width 0.25) (layer F.Cu) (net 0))
 (segment (start 134.0398 136.402) (end 134.366 136.7282) (width 0.25) (layer F.Cu) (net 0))
 (segment (start 133.3898 135.0486) (end 133.3898 136.387) (width 0.25) (layer F.Cu) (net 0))
 (segment (start 138.4554 137.6426) (end 140.0048 139.192) (width 0.25) (layer F.Cu) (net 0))
 (segment (start 136.5504 137.6426) (end 138.4554 137.6426) (width 0.25) (layer F.Cu) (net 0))
 (segment (start 136.0932 137.1854) (end 136.5504 137.6426) (width 0.25) (layer F.Cu) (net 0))
 (segment (start 134.1882 137.1854) (end 136.0932 137.1854) (width 0.25) (layer F.Cu) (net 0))
 (segment (start 133.3898 136.387) (end 134.1882 137.1854) (width 0.25) (layer F.Cu) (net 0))
 (segment (start 132.7398 135.0486) (end 132.7398 136.372) (width 0.25) (layer F.Cu) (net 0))
 (segment (start 135.9154 137.6426) (end 137.4648 139.192) (width 0.25) (layer F.Cu) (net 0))
 (segment (start 134.0104 137.6426) (end 135.9154 137.6426) (width 0.25) (layer F.Cu) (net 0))
 (segment (start 132.7398 136.372) (end 134.0104 137.6426) (width 0.25) (layer F.Cu) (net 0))
 (segment (start 130.1398 135.0486) (end 130.1398 136.357) (width 0.25) (layer F.Cu) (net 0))
 (segment (start 130.1398 136.357) (end 127.3048 139.192) (width 0.25) (layer F.Cu) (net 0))
 (segment (start 132.0898 135.0486) (end 132.0898 136.357) (width 0.25) (layer F.Cu) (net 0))
 (segment (start 132.0898 136.357) (end 134.9248 139.192) (width 0.25) (layer F.Cu) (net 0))
 (segment (start 130.7898 135.0486) (end 130.7898 138.247) (width 0.25) (layer F.Cu) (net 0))
 (segment (start 130.7898 138.247) (end 129.8448 139.192) (width 0.25) (layer F.Cu) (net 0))
 (segment (start 131.4398 135.0486) (end 131.4398 138.247) (width 0.25) (layer F.Cu) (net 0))
 (segment (start 131.4398 138.247) (end 132.3848 139.192) (width 0.25) (layer F.Cu) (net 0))
 (segment (start 128.8398 128.2986) (end 128.8398 126.9602) (width 0.25) (layer F.Cu) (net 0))
 (segment (start 123.7742 125.7046) (end 122.2248 124.1552) (width 0.25) (layer F.Cu) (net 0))
 (segment (start 125.6792 125.7046) (end 123.7742 125.7046) (width 0.25) (layer F.Cu) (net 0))
 (segment (start 126.1364 126.1618) (end 125.6792 125.7046) (width 0.25) (layer F.Cu) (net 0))
 (segment (start 128.0414 126.1618) (end 126.1364 126.1618) (width 0.25) (layer F.Cu) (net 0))
 (segment (start 128.8398 126.9602) (end 128.0414 126.1618) (width 0.25) (layer F.Cu) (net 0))
 (segment (start 129.4898 128.2986) (end 129.4898 126.9752) (width 0.25) (layer F.Cu) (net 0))
 (segment (start 126.3142 125.7046) (end 124.7648 124.1552) (width 0.25) (layer F.Cu) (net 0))
 (segment (start 128.2192 125.7046) (end 126.3142 125.7046) (width 0.25) (layer F.Cu) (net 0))
 (segment (start 129.4898 126.9752) (end 128.2192 125.7046) (width 0.25) (layer F.Cu) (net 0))
 (segment (start 130.1398 128.2986) (end 130.1398 126.9902) (width 0.25) (layer F.Cu) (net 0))
 (segment (start 130.1398 126.9902) (end 127.3048 124.1552) (width 0.25) (layer F.Cu) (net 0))
 (segment (start 130.7898 128.2986) (end 130.7898 125.1002) (width 0.25) (layer F.Cu) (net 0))
 (segment (start 130.7898 125.1002) (end 129.8448 124.1552) (width 0.25) (layer F.Cu) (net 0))
 (segment (start 134.6898 128.2986) (end 134.6898 127.0572) (width 0.25) (layer F.Cu) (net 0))
 (segment (start 143.5354 125.7046) (end 145.0848 124.1552) (width 0.25) (layer F.Cu) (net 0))
 (segment (start 141.6304 125.7046) (end 143.5354 125.7046) (width 0.25) (layer F.Cu) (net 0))
 (segment (start 141.1732 126.1618) (end 141.6304 125.7046) (width 0.25) (layer F.Cu) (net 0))
 (segment (start 139.2682 126.1618) (end 141.1732 126.1618) (width 0.25) (layer F.Cu) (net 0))
 (segment (start 138.811 126.619) (end 139.2682 126.1618) (width 0.25) (layer F.Cu) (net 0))
 (segment (start 136.906 126.619) (end 138.811 126.619) (width 0.25) (layer F.Cu) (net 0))
 (segment (start 136.4488 127.0762) (end 136.906 126.619) (width 0.25) (layer F.Cu) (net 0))
 (segment (start 134.7088 127.0762) (end 136.4488 127.0762) (width 0.25) (layer F.Cu) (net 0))
 (segment (start 134.6898 127.0572) (end 134.7088 127.0762) (width 0.25) (layer F.Cu) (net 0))
 (segment (start 134.0398 128.2986) (end 134.0398 126.9452) (width 0.25) (layer F.Cu) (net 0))
 (segment (start 140.9954 125.7046) (end 142.5448 124.1552) (width 0.25) (layer F.Cu) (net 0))
 (segment (start 139.0904 125.7046) (end 140.9954 125.7046) (width 0.25) (layer F.Cu) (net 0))
 (segment (start 138.6332 126.1618) (end 139.0904 125.7046) (width 0.25) (layer F.Cu) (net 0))
 (segment (start 136.7282 126.1618) (end 138.6332 126.1618) (width 0.25) (layer F.Cu) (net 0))
 (segment (start 136.271 126.619) (end 136.7282 126.1618) (width 0.25) (layer F.Cu) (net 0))
 (segment (start 134.366 126.619) (end 136.271 126.619) (width 0.25) (layer F.Cu) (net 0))
 (segment (start 134.0398 126.9452) (end 134.366 126.619) (width 0.25) (layer F.Cu) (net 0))
 (segment (start 133.3898 128.2986) (end 133.3898 126.9602) (width 0.25) (layer F.Cu) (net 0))
 (segment (start 138.4554 125.7046) (end 140.0048 124.1552) (width 0.25) (layer F.Cu) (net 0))
 (segment (start 136.5504 125.7046) (end 138.4554 125.7046) (width 0.25) (layer F.Cu) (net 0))
 (segment (start 136.0932 126.1618) (end 136.5504 125.7046) (width 0.25) (layer F.Cu) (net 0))
 (segment (start 134.1882 126.1618) (end 136.0932 126.1618) (width 0.25) (layer F.Cu) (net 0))
 (segment (start 133.3898 126.9602) (end 134.1882 126.1618) (width 0.25) (layer F.Cu) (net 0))
 (segment (start 132.7398 128.2986) (end 132.7398 126.9752) (width 0.25) (layer F.Cu) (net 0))
 (segment (start 135.9154 125.7046) (end 137.4648 124.1552) (width 0.25) (layer F.Cu) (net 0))
 (segment (start 134.0104 125.7046) (end 135.9154 125.7046) (width 0.25) (layer F.Cu) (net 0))
 (segment (start 132.7398 126.9752) (end 134.0104 125.7046) (width 0.25) (layer F.Cu) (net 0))
 (segment (start 132.0898 128.2986) (end 132.0898 126.9902) (width 0.25) (layer F.Cu) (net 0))
 (segment (start 132.0898 126.9902) (end 134.9248 124.1552) (width 0.25) (layer F.Cu) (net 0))
 (segment (start 131.4398 128.2986) (end 131.4398 125.1002) (width 0.25) (layer F.Cu) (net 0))
 (segment (start 131.4398 125.1002) (end 132.3848 124.1552) (width 0.25) (layer F.Cu) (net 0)))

